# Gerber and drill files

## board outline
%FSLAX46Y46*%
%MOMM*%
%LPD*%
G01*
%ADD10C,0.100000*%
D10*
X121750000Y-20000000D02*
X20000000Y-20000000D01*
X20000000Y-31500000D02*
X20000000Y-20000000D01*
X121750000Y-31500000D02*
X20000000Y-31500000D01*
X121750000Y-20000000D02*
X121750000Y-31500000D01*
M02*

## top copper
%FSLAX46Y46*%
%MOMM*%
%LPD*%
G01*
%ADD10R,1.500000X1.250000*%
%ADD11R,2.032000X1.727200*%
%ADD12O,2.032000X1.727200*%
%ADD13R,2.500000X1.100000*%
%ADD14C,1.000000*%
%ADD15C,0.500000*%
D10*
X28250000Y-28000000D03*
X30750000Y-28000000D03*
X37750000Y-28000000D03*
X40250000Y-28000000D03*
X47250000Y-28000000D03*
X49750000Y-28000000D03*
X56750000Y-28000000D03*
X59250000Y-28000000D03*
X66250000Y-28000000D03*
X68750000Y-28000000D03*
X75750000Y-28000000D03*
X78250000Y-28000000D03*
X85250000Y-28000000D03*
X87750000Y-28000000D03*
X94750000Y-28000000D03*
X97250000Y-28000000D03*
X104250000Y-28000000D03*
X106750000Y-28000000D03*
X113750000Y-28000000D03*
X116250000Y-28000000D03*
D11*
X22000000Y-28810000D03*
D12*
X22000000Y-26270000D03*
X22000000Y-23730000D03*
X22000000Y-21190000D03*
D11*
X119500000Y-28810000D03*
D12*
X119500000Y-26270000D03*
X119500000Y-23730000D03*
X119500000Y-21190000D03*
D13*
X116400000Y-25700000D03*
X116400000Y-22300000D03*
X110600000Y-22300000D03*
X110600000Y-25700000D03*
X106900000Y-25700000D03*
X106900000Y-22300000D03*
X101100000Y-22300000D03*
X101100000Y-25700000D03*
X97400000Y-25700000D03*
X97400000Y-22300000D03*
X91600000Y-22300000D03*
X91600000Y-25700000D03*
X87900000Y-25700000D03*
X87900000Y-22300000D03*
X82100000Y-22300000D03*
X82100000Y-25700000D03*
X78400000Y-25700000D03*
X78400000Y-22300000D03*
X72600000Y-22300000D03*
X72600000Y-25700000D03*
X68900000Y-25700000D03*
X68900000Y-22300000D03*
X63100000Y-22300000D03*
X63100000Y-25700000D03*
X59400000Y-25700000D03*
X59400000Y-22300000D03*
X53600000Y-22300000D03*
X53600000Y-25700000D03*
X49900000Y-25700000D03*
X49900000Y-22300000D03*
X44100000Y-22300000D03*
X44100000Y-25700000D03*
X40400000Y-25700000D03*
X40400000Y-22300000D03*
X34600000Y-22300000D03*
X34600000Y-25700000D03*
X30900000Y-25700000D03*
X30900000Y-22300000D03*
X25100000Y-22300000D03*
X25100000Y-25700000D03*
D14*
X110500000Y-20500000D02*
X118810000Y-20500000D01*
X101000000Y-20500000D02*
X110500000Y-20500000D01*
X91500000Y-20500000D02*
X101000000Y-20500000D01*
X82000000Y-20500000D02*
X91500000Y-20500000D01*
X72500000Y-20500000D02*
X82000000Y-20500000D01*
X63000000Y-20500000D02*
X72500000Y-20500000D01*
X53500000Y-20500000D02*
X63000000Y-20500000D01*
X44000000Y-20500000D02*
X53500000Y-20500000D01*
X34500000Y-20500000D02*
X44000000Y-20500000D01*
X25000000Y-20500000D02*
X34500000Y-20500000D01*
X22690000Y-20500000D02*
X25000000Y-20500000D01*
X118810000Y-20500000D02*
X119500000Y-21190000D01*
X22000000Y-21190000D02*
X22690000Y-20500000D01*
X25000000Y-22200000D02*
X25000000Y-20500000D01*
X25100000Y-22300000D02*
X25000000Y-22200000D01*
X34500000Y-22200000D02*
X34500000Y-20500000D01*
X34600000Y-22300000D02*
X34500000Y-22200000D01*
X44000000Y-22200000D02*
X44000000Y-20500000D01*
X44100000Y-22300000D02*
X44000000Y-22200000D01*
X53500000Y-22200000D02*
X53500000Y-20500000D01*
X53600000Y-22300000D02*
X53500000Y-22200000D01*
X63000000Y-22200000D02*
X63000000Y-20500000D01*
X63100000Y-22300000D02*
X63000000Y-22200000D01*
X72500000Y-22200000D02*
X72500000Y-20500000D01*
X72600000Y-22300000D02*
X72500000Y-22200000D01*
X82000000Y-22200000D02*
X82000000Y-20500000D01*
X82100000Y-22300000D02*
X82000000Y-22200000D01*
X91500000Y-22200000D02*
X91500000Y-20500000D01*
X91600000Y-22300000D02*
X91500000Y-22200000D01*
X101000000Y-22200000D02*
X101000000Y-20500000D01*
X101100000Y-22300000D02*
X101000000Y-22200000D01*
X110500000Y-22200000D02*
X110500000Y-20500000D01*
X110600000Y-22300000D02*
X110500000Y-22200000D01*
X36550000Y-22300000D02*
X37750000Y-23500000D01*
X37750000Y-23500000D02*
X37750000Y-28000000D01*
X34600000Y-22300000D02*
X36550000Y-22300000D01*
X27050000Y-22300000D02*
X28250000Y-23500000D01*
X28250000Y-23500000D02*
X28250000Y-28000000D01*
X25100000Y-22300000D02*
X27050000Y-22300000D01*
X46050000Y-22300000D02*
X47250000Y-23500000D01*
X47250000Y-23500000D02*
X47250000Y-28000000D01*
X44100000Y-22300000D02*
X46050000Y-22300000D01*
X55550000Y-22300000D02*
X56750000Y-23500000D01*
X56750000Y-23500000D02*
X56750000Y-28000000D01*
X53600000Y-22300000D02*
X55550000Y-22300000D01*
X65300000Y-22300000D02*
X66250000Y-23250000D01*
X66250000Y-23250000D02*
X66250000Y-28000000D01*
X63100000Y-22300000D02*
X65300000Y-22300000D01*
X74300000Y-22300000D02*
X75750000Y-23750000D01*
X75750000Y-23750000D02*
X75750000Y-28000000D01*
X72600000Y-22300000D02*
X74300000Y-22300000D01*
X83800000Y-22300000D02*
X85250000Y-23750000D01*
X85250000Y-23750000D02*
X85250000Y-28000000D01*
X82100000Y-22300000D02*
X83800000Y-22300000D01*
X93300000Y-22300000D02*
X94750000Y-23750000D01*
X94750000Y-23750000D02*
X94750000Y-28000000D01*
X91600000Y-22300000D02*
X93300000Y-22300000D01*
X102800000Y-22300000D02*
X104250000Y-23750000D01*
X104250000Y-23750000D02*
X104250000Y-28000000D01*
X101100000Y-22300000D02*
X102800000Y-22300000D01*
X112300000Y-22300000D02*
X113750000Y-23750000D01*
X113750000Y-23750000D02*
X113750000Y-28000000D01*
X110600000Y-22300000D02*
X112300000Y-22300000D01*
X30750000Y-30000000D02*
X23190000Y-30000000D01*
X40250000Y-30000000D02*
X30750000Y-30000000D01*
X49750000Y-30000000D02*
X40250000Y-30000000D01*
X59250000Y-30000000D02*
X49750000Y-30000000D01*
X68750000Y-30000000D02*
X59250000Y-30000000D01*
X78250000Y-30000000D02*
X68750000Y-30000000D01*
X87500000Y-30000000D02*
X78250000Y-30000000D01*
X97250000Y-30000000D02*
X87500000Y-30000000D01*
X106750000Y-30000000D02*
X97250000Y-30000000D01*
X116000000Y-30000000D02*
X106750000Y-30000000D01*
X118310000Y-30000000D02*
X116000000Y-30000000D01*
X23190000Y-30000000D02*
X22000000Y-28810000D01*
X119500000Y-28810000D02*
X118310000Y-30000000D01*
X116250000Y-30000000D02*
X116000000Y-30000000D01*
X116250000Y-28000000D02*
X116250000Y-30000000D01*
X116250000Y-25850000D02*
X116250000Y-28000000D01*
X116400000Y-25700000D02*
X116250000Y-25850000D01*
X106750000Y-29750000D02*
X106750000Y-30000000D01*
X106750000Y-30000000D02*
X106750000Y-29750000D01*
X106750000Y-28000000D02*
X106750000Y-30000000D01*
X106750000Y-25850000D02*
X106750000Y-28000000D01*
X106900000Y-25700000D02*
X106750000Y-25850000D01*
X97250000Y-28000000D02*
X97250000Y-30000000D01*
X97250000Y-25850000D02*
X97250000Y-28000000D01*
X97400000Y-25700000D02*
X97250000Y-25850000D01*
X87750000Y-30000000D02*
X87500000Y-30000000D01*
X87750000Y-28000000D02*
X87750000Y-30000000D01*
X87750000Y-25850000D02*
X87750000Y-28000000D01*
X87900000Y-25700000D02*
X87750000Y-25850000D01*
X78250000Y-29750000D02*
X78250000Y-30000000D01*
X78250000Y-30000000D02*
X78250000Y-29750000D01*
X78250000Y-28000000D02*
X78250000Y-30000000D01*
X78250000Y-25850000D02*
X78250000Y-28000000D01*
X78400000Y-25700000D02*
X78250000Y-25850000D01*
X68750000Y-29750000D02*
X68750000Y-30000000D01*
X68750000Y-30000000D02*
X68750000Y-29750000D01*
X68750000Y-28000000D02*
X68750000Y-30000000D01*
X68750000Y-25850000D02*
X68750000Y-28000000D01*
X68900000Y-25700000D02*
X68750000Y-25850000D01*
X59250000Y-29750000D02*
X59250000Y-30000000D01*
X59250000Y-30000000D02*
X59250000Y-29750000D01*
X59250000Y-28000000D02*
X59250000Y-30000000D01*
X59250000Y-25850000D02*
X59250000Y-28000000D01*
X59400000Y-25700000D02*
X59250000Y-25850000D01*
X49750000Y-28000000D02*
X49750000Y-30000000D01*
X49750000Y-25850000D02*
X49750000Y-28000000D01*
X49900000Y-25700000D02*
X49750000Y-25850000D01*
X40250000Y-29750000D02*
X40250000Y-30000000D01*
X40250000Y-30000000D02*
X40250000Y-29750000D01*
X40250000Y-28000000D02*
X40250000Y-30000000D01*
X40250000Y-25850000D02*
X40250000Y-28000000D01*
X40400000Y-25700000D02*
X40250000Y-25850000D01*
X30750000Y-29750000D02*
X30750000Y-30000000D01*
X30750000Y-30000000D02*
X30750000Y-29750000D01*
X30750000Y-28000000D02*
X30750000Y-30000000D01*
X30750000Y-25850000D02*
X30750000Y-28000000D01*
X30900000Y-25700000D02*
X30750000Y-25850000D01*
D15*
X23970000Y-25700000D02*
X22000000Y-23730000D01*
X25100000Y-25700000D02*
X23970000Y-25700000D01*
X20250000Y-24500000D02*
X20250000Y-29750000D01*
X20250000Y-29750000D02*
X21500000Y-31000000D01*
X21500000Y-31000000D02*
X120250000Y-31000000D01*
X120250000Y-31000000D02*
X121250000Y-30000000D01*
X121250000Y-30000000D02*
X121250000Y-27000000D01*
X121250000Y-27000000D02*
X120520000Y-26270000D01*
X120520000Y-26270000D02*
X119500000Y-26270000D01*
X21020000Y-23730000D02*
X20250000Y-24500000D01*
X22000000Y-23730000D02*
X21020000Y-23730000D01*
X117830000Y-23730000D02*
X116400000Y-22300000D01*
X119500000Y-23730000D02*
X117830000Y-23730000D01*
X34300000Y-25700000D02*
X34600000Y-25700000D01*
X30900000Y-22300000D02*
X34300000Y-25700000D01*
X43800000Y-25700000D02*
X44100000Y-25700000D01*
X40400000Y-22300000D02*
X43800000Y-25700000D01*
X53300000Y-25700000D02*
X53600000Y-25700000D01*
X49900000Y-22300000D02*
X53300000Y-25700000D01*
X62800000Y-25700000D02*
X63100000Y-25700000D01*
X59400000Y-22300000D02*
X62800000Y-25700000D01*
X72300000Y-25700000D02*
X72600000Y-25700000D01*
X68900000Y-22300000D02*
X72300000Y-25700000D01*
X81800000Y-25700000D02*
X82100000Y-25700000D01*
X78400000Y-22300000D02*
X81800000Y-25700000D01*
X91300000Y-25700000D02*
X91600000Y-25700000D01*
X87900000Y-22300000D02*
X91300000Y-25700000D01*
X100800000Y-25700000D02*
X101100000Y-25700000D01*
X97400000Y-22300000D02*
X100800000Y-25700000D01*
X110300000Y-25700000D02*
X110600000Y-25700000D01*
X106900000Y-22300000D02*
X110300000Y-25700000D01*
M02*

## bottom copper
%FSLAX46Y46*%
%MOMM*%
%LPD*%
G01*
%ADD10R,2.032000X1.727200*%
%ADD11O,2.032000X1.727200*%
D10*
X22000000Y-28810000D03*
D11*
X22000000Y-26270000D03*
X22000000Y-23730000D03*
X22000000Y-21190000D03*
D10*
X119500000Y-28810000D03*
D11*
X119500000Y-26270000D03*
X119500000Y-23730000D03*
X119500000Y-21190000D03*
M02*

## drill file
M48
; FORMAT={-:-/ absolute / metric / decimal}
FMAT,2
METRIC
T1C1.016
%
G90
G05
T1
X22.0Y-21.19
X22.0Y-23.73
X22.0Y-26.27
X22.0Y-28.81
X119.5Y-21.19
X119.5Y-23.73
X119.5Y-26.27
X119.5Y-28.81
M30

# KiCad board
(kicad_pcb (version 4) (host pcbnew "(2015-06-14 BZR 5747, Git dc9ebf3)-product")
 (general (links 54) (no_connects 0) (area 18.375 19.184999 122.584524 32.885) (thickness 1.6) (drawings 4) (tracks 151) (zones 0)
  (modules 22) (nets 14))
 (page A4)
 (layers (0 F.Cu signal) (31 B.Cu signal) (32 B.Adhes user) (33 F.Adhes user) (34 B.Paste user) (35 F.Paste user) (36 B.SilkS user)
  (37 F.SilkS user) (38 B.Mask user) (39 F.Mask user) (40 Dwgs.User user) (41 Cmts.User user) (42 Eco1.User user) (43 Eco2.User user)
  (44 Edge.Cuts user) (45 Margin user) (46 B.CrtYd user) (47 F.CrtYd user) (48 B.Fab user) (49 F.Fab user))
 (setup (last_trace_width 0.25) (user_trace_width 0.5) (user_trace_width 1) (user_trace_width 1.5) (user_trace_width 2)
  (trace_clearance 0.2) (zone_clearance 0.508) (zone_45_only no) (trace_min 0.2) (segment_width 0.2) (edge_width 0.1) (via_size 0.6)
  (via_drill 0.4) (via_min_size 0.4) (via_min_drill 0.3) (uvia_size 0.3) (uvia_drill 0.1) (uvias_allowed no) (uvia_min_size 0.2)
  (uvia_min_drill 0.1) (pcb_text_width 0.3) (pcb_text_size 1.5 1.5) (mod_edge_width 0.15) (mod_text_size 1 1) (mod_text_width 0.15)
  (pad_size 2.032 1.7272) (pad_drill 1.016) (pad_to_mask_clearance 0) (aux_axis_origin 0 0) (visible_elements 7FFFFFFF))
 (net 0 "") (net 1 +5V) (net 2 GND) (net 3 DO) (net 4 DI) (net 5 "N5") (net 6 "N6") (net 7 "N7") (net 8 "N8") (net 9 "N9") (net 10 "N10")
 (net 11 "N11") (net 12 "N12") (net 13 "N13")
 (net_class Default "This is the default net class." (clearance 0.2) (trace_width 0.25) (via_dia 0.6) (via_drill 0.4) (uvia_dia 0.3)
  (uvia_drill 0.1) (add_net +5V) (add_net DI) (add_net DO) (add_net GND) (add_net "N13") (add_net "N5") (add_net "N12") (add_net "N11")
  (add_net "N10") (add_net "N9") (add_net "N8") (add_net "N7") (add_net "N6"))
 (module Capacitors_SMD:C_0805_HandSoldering (layer F.Cu) (at 29.5 28)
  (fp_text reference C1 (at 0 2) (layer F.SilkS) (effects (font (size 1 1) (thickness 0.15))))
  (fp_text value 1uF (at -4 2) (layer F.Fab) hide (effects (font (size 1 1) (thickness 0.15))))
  (pad 1 smd rect (at -1.25 0) (size 1.5 1.25) (layers F.Cu F.Paste F.Mask) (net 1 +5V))
  (pad 2 smd rect (at 1.25 0) (size 1.5 1.25) (layers F.Cu F.Paste F.Mask) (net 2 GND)))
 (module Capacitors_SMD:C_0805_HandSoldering (layer F.Cu) (at 39 28)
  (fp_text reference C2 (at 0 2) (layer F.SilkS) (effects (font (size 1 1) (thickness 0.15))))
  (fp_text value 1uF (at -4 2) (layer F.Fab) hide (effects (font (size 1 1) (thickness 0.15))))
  (pad 1 smd rect (at -1.25 0) (size 1.5 1.25) (layers F.Cu F.Paste F.Mask) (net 1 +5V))
  (pad 2 smd rect (at 1.25 0) (size 1.5 1.25) (layers F.Cu F.Paste F.Mask) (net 2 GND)))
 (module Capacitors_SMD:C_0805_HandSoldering (layer F.Cu) (at 48.5 28)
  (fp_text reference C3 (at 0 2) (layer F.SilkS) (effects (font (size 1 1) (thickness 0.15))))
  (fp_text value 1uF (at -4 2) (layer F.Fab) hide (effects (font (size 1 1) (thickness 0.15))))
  (pad 1 smd rect (at -1.25 0) (size 1.5 1.25) (layers F.Cu F.Paste F.Mask) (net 1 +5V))
  (pad 2 smd rect (at 1.25 0) (size 1.5 1.25) (layers F.Cu F.Paste F.Mask) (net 2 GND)))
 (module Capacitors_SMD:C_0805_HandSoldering (layer F.Cu) (at 58 28)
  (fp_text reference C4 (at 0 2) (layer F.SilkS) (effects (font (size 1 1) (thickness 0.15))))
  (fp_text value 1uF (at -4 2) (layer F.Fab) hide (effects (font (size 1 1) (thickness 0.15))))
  (pad 1 smd rect (at -1.25 0) (size 1.5 1.25) (layers F.Cu F.Paste F.Mask) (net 1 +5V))
  (pad 2 smd rect (at 1.25 0) (size 1.5 1.25) (layers F.Cu F.Paste F.Mask) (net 2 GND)))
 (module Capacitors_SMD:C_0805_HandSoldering (layer F.Cu) (at 67.5 28)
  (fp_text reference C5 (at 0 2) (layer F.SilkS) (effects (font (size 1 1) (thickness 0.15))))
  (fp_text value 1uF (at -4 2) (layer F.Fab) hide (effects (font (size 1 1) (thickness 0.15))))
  (pad 1 smd rect (at -1.25 0) (size 1.5 1.25) (layers F.Cu F.Paste F.Mask) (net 1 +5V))
  (pad 2 smd rect (at 1.25 0) (size 1.5 1.25) (layers F.Cu F.Paste F.Mask) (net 2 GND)))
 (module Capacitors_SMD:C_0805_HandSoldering (layer F.Cu) (at 77 28)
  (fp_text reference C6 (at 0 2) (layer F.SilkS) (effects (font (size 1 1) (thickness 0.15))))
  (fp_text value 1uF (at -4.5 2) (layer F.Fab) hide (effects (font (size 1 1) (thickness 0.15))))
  (pad 1 smd rect (at -1.25 0) (size 1.5 1.25) (layers F.Cu F.Paste F.Mask) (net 1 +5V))
  (pad 2 smd rect (at 1.25 0) (size 1.5 1.25) (layers F.Cu F.Paste F.Mask) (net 2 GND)))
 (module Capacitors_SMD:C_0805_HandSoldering (layer F.Cu) (at 86.5 28)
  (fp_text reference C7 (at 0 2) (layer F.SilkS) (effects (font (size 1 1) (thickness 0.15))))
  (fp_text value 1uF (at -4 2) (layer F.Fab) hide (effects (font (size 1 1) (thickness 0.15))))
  (pad 1 smd rect (at -1.25 0) (size 1.5 1.25) (layers F.Cu F.Paste F.Mask) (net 1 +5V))
  (pad 2 smd rect (at 1.25 0) (size 1.5 1.25) (layers F.Cu F.Paste F.Mask) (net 2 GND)))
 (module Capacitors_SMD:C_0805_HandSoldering (layer F.Cu) (at 96 28)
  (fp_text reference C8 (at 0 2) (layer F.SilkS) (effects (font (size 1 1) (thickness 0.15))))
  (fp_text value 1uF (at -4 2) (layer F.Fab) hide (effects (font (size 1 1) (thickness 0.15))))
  (pad 1 smd rect (at -1.25 0) (size 1.5 1.25) (layers F.Cu F.Paste F.Mask) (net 1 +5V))
  (pad 2 smd rect (at 1.25 0) (size 1.5 1.25) (layers F.Cu F.Paste F.Mask) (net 2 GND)))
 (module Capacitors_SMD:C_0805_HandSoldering (layer F.Cu) (at 105.5 28)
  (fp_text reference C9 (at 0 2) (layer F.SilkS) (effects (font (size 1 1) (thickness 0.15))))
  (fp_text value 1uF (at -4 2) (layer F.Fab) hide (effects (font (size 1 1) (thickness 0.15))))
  (pad 1 smd rect (at -1.25 0) (size 1.5 1.25) (layers F.Cu F.Paste F.Mask) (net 1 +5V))
  (pad 2 smd rect (at 1.25 0) (size 1.5 1.25) (layers F.Cu F.Paste F.Mask) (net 2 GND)))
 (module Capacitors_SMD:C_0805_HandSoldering (layer F.Cu) (at 115 28)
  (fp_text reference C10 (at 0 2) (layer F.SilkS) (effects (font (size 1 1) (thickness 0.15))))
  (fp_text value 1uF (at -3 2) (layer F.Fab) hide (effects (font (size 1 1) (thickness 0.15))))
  (pad 1 smd rect (at -1.25 0) (size 1.5 1.25) (layers F.Cu F.Paste F.Mask) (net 1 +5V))
  (pad 2 smd rect (at 1.25 0) (size 1.5 1.25) (layers F.Cu F.Paste F.Mask) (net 2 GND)))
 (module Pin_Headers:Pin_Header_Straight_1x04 (layer F.Cu) (at 22 28.81 180)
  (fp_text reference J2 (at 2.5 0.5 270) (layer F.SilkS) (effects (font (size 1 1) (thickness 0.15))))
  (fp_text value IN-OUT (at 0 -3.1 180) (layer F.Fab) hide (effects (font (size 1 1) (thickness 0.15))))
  (pad 1 thru_hole rect (at 0 0 180) (size 2.032 1.7272) (drill 1.016) (layers *.Cu *.Mask F.SilkS) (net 2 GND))
  (pad 2 thru_hole oval (at 0 2.54 180) (size 2.032 1.7272) (drill 1.016) (layers *.Cu *.Mask F.SilkS))
  (pad 3 thru_hole oval (at 0 5.08 180) (size 2.032 1.7272) (drill 1.016) (layers *.Cu *.Mask F.SilkS) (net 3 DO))
  (pad 4 thru_hole oval (at 0 7.62 180) (size 2.032 1.7272) (drill 1.016) (layers *.Cu *.Mask F.SilkS) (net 1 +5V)))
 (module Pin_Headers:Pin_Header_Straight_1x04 (layer F.Cu) (at 119.5 28.81 180)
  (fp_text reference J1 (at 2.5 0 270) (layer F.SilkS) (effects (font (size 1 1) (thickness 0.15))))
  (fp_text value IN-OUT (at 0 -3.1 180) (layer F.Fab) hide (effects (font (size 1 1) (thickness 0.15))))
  (pad 1 thru_hole rect (at 0 0 180) (size 2.032 1.7272) (drill 1.016) (layers *.Cu *.Mask F.SilkS) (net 2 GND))
  (pad 2 thru_hole oval (at 0 2.54 180) (size 2.032 1.7272) (drill 1.016) (layers *.Cu *.Mask F.SilkS) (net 3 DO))
  (pad 3 thru_hole oval (at 0 5.08 180) (size 2.032 1.7272) (drill 1.016) (layers *.Cu *.Mask F.SilkS) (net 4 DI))
  (pad 4 thru_hole oval (at 0 7.62 180) (size 2.032 1.7272) (drill 1.016) (layers *.Cu *.Mask F.SilkS) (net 1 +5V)))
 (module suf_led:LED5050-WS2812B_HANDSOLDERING (layer F.Cu) (at 113.5 24 90)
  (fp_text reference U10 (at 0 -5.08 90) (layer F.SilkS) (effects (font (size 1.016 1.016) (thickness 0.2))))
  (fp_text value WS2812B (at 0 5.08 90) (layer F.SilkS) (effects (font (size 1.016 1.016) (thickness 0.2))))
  (pad 3 smd rect (at -1.7 2.9 90) (size 1.1 2.5) (layers F.Cu F.Paste F.Mask) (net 2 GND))
  (pad 4 smd rect (at 1.7 2.9 90) (size 1.1 2.5) (layers F.Cu F.Paste F.Mask) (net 4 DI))
  (pad 1 smd rect (at 1.7 -2.9 90) (size 1.1 2.5) (layers F.Cu F.Paste F.Mask) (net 1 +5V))
  (pad 2 smd rect (at -1.7 -2.9 90) (size 1.1 2.5) (layers F.Cu F.Paste F.Mask) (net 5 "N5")))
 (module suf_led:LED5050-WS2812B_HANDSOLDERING (layer F.Cu) (at 104 24 90)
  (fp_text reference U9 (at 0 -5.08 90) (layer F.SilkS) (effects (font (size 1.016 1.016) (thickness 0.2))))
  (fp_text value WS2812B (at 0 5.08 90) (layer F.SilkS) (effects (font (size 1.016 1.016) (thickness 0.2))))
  (pad 3 smd rect (at -1.7 2.9 90) (size 1.1 2.5) (layers F.Cu F.Paste F.Mask) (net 2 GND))
  (pad 4 smd rect (at 1.7 2.9 90) (size 1.1 2.5) (layers F.Cu F.Paste F.Mask) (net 5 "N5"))
  (pad 1 smd rect (at 1.7 -2.9 90) (size 1.1 2.5) (layers F.Cu F.Paste F.Mask) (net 1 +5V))
  (pad 2 smd rect (at -1.7 -2.9 90) (size 1.1 2.5) (layers F.Cu F.Paste F.Mask) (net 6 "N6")))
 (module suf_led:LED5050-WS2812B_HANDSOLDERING (layer F.Cu) (at 94.5 24 90)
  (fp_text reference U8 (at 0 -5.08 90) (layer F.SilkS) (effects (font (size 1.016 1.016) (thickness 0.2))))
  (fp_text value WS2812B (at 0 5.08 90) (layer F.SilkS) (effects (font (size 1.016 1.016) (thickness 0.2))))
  (pad 3 smd rect (at -1.7 2.9 90) (size 1.1 2.5) (layers F.Cu F.Paste F.Mask) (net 2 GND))
  (pad 4 smd rect (at 1.7 2.9 90) (size 1.1 2.5) (layers F.Cu F.Paste F.Mask) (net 6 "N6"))
  (pad 1 smd rect (at 1.7 -2.9 90) (size 1.1 2.5) (layers F.Cu F.Paste F.Mask) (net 1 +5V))
  (pad 2 smd rect (at -1.7 -2.9 90) (size 1.1 2.5) (layers F.Cu F.Paste F.Mask) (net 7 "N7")))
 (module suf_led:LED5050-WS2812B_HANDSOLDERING (layer F.Cu) (at 85 24 90)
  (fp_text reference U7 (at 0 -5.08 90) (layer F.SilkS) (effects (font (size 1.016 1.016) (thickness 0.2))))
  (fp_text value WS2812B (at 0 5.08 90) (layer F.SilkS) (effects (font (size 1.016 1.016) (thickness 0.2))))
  (pad 3 smd rect (at -1.7 2.9 90) (size 1.1 2.5) (layers F.Cu F.Paste F.Mask) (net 2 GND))
  (pad 4 smd rect (at 1.7 2.9 90) (size 1.1 2.5) (layers F.Cu F.Paste F.Mask) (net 7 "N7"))
  (pad 1 smd rect (at 1.7 -2.9 90) (size 1.1 2.5) (layers F.Cu F.Paste F.Mask) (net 1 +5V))
  (pad 2 smd rect (at -1.7 -2.9 90) (size 1.1 2.5) (layers F.Cu F.Paste F.Mask) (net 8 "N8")))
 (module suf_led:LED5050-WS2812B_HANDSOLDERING (layer F.Cu) (at 75.5 24 90)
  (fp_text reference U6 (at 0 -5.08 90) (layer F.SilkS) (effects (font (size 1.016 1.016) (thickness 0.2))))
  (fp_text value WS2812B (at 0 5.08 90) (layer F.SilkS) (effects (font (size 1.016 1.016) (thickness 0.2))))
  (pad 3 smd rect (at -1.7 2.9 90) (size 1.1 2.5) (layers F.Cu F.Paste F.Mask) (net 2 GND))
  (pad 4 smd rect (at 1.7 2.9 90) (size 1.1 2.5) (layers F.Cu F.Paste F.Mask) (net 8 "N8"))
  (pad 1 smd rect (at 1.7 -2.9 90) (size 1.1 2.5) (layers F.Cu F.Paste F.Mask) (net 1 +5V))
  (pad 2 smd rect (at -1.7 -2.9 90) (size 1.1 2.5) (layers F.Cu F.Paste F.Mask) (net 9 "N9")))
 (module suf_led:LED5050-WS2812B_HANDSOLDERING (layer F.Cu) (at 66 24 90)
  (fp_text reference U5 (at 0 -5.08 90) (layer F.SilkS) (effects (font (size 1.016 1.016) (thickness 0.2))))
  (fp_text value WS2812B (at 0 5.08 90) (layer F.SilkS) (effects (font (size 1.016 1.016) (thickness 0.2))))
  (pad 3 smd rect (at -1.7 2.9 90) (size 1.1 2.5) (layers F.Cu F.Paste F.Mask) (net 2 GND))
  (pad 4 smd rect (at 1.7 2.9 90) (size 1.1 2.5) (layers F.Cu F.Paste F.Mask) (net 9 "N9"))
  (pad 1 smd rect (at 1.7 -2.9 90) (size 1.1 2.5) (layers F.Cu F.Paste F.Mask) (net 1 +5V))
  (pad 2 smd rect (at -1.7 -2.9 90) (size 1.1 2.5) (layers F.Cu F.Paste F.Mask) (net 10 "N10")))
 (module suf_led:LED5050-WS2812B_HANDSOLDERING (layer F.Cu) (at 56.5 24 90)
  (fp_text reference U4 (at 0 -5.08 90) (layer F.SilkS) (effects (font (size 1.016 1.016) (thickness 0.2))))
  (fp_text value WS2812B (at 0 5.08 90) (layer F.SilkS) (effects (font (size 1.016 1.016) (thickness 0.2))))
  (pad 3 smd rect (at -1.7 2.9 90) (size 1.1 2.5) (layers F.Cu F.Paste F.Mask) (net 2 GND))
  (pad 4 smd rect (at 1.7 2.9 90) (size 1.1 2.5) (layers F.Cu F.Paste F.Mask) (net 10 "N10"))
  (pad 1 smd rect (at 1.7 -2.9 90) (size 1.1 2.5) (layers F.Cu F.Paste F.Mask) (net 1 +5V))
  (pad 2 smd rect (at -1.7 -2.9 90) (size 1.1 2.5) (layers F.Cu F.Paste F.Mask) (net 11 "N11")))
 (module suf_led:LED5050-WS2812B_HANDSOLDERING (layer F.Cu) (at 47 24 90)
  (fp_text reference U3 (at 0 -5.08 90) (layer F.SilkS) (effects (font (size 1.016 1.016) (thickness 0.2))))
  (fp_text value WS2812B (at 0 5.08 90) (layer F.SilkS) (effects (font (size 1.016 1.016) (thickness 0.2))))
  (pad 3 smd rect (at -1.7 2.9 90) (size 1.1 2.5) (layers F.Cu F.Paste F.Mask) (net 2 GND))
  (pad 4 smd rect (at 1.7 2.9 90) (size 1.1 2.5) (layers F.Cu F.Paste F.Mask) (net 11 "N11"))
  (pad 1 smd rect (at 1.7 -2.9 90) (size 1.1 2.5) (layers F.Cu F.Paste F.Mask) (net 1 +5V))
  (pad 2 smd rect (at -1.7 -2.9 90) (size 1.1 2.5) (layers F.Cu F.Paste F.Mask) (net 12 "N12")))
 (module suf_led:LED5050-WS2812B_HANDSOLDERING (layer F.Cu) (at 37.5 24 90)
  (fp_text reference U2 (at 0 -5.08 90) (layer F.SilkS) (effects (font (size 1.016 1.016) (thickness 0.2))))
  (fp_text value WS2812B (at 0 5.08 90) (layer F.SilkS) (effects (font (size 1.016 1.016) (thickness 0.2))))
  (pad 3 smd rect (at -1.7 2.9 90) (size 1.1 2.5) (layers F.Cu F.Paste F.Mask) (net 2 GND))
  (pad 4 smd rect (at 1.7 2.9 90) (size 1.1 2.5) (layers F.Cu F.Paste F.Mask) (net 12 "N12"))
  (pad 1 smd rect (at 1.7 -2.9 90) (size 1.1 2.5) (layers F.Cu F.Paste F.Mask) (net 1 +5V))
  (pad 2 smd rect (at -1.7 -2.9 90) (size 1.1 2.5) (layers F.Cu F.Paste F.Mask) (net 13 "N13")))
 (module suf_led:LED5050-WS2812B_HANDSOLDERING (layer F.Cu) (at 28 24 90)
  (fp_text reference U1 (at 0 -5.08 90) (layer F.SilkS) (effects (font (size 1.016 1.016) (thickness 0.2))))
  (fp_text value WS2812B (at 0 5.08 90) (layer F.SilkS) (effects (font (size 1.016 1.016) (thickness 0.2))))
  (pad 3 smd rect (at -1.7 2.9 90) (size 1.1 2.5) (layers F.Cu F.Paste F.Mask) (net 2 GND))
  (pad 4 smd rect (at 1.7 2.9 90) (size 1.1 2.5) (layers F.Cu F.Paste F.Mask) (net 13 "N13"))
  (pad 1 smd rect (at 1.7 -2.9 90) (size 1.1 2.5) (layers F.Cu F.Paste F.Mask) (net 1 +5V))
  (pad 2 smd rect (at -1.7 -2.9 90) (size 1.1 2.5) (layers F.Cu F.Paste F.Mask) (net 3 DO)))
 (gr_line (start 121.75 20) (end 20 20) (angle 90) (layer Edge.Cuts) (width 0.1))
 (gr_line (start 20 31.5) (end 20 20) (angle 90) (layer Edge.Cuts) (width 0.1))
 (gr_line (start 121.75 31.5) (end 20 31.5) (angle 90) (layer Edge.Cuts) (width 0.1))
 (gr_line (start 121.75 20) (end 121.75 31.5) (angle 90) (layer Edge.Cuts) (width 0.1))
 (segment (start 110.5 20.5) (end 118.81 20.5) (width 1) (layer F.Cu) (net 1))
 (segment (start 101 20.5) (end 110.5 20.5) (width 1) (layer F.Cu) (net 1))
 (segment (start 91.5 20.5) (end 101 20.5) (width 1) (layer F.Cu) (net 1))
 (segment (start 82 20.5) (end 91.5 20.5) (width 1) (layer F.Cu) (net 1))
 (segment (start 72.5 20.5) (end 82 20.5) (width 1) (layer F.Cu) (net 1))
 (segment (start 63 20.5) (end 72.5 20.5) (width 1) (layer F.Cu) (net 1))
 (segment (start 53.5 20.5) (end 63 20.5) (width 1) (layer F.Cu) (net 1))
 (segment (start 44 20.5) (end 53.5 20.5) (width 1) (layer F.Cu) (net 1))
 (segment (start 34.5 20.5) (end 44 20.5) (width 1) (layer F.Cu) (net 1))
 (segment (start 25 20.5) (end 34.5 20.5) (width 1) (layer F.Cu) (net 1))
 (segment (start 22.69 20.5) (end 25 20.5) (width 1) (layer F.Cu) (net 1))
 (segment (start 118.81 20.5) (end 119.5 21.19) (width 1) (layer F.Cu) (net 1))
 (segment (start 22 21.19) (end 22.69 20.5) (width 1) (layer F.Cu) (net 1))
 (segment (start 25 22.2) (end 25 20.5) (width 1) (layer F.Cu) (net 1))
 (segment (start 25.1 22.3) (end 25 22.2) (width 1) (layer F.Cu) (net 1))
 (segment (start 34.5 22.2) (end 34.5 20.5) (width 1) (layer F.Cu) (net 1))
 (segment (start 34.6 22.3) (end 34.5 22.2) (width 1) (layer F.Cu) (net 1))
 (segment (start 44 22.2) (end 44 20.5) (width 1) (layer F.Cu) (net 1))
 (segment (start 44.1 22.3) (end 44 22.2) (width 1) (layer F.Cu) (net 1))
 (segment (start 53.5 22.2) (end 53.5 20.5) (width 1) (layer F.Cu) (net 1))
 (segment (start 53.6 22.3) (end 53.5 22.2) (width 1) (layer F.Cu) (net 1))
 (segment (start 63 22.2) (end 63 20.5) (width 1) (layer F.Cu) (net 1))
 (segment (start 63.1 22.3) (end 63 22.2) (width 1) (layer F.Cu) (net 1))
 (segment (start 72.5 22.2) (end 72.5 20.5) (width 1) (layer F.Cu) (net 1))
 (segment (start 72.6 22.3) (end 72.5 22.2) (width 1) (layer F.Cu) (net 1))
 (segment (start 82 22.2) (end 82 20.5) (width 1) (layer F.Cu) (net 1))
 (segment (start 82.1 22.3) (end 82 22.2) (width 1) (layer F.Cu) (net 1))
 (segment (start 91.5 22.2) (end 91.5 20.5) (width 1) (layer F.Cu) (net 1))
 (segment (start 91.6 22.3) (end 91.5 22.2) (width 1) (layer F.Cu) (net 1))
 (segment (start 101 22.2) (end 101 20.5) (width 1) (layer F.Cu) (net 1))
 (segment (start 101.1 22.3) (end 101 22.2) (width 1) (layer F.Cu) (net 1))
 (segment (start 110.5 22.2) (end 110.5 20.5) (width 1) (layer F.Cu) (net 1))
 (segment (start 110.6 22.3) (end 110.5 22.2) (width 1) (layer F.Cu) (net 1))
 (segment (start 36.55 22.3) (end 37.75 23.5) (width 1) (layer F.Cu) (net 1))
 (segment (start 37.75 23.5) (end 37.75 28) (width 1) (layer F.Cu) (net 1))
 (segment (start 34.6 22.3) (end 36.55 22.3) (width 1) (layer F.Cu) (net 1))
 (segment (start 27.05 22.3) (end 28.25 23.5) (width 1) (layer F.Cu) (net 1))
 (segment (start 28.25 23.5) (end 28.25 28) (width 1) (layer F.Cu) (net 1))
 (segment (start 25.1 22.3) (end 27.05 22.3) (width 1) (layer F.Cu) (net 1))
 (segment (start 46.05 22.3) (end 47.25 23.5) (width 1) (layer F.Cu) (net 1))
 (segment (start 47.25 23.5) (end 47.25 28) (width 1) (layer F.Cu) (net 1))
 (segment (start 44.1 22.3) (end 46.05 22.3) (width 1) (layer F.Cu) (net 1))
 (segment (start 55.55 22.3) (end 56.75 23.5) (width 1) (layer F.Cu) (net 1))
 (segment (start 56.75 23.5) (end 56.75 28) (width 1) (layer F.Cu) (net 1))
 (segment (start 53.6 22.3) (end 55.55 22.3) (width 1) (layer F.Cu) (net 1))
 (segment (start 65.3 22.3) (end 66.25 23.25) (width 1) (layer F.Cu) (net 1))
 (segment (start 66.25 23.25) (end 66.25 28) (width 1) (layer F.Cu) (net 1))
 (segment (start 63.1 22.3) (end 65.3 22.3) (width 1) (layer F.Cu) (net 1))
 (segment (start 74.3 22.3) (end 75.75 23.75) (width 1) (layer F.Cu) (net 1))
 (segment (start 75.75 23.75) (end 75.75 28) (width 1) (layer F.Cu) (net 1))
 (segment (start 72.6 22.3) (end 74.3 22.3) (width 1) (layer F.Cu) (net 1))
 (segment (start 83.8 22.3) (end 85.25 23.75) (width 1) (layer F.Cu) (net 1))
 (segment (start 85.25 23.75) (end 85.25 28) (width 1) (layer F.Cu) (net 1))
 (segment (start 82.1 22.3) (end 83.8 22.3) (width 1) (layer F.Cu) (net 1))
 (segment (start 93.3 22.3) (end 94.75 23.75) (width 1) (layer F.Cu) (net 1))
 (segment (start 94.75 23.75) (end 94.75 28) (width 1) (layer F.Cu) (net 1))
 (segment (start 91.6 22.3) (end 93.3 22.3) (width 1) (layer F.Cu) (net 1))
 (segment (start 102.8 22.3) (end 104.25 23.75) (width 1) (layer F.Cu) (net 1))
 (segment (start 104.25 23.75) (end 104.25 28) (width 1) (layer F.Cu) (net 1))
 (segment (start 101.1 22.3) (end 102.8 22.3) (width 1) (layer F.Cu) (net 1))
 (segment (start 112.3 22.3) (end 113.75 23.75) (width 1) (layer F.Cu) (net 1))
 (segment (start 113.75 23.75) (end 113.75 28) (width 1) (layer F.Cu) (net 1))
 (segment (start 110.6 22.3) (end 112.3 22.3) (width 1) (layer F.Cu) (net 1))
 (segment (start 30.75 30) (end 23.19 30) (width 1) (layer F.Cu) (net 2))
 (segment (start 40.25 30) (end 30.75 30) (width 1) (layer F.Cu) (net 2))
 (segment (start 49.75 30) (end 40.25 30) (width 1) (layer F.Cu) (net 2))
 (segment (start 59.25 30) (end 49.75 30) (width 1) (layer F.Cu) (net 2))
 (segment (start 68.75 30) (end 59.25 30) (width 1) (layer F.Cu) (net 2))
 (segment (start 78.25 30) (end 68.75 30) (width 1) (layer F.Cu) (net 2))
 (segment (start 87.5 30) (end 78.25 30) (width 1) (layer F.Cu) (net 2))
 (segment (start 97.25 30) (end 87.5 30) (width 1) (layer F.Cu) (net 2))
 (segment (start 106.75 30) (end 97.25 30) (width 1) (layer F.Cu) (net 2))
 (segment (start 116 30) (end 106.75 30) (width 1) (layer F.Cu) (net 2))
 (segment (start 118.31 30) (end 116 30) (width 1) (layer F.Cu) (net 2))
 (segment (start 23.19 30) (end 22 28.81) (width 1) (layer F.Cu) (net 2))
 (segment (start 119.5 28.81) (end 118.31 30) (width 1) (layer F.Cu) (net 2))
 (segment (start 116.25 30) (end 116 30) (width 1) (layer F.Cu) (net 2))
 (segment (start 116.25 28) (end 116.25 30) (width 1) (layer F.Cu) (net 2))
 (segment (start 116.25 25.85) (end 116.25 28) (width 1) (layer F.Cu) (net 2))
 (segment (start 116.4 25.7) (end 116.25 25.85) (width 1) (layer F.Cu) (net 2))
 (segment (start 106.75 29.75) (end 106.75 30) (width 1) (layer F.Cu) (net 2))
 (segment (start 106.75 30) (end 106.75 29.75) (width 1) (layer F.Cu) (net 2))
 (segment (start 106.75 28) (end 106.75 30) (width 1) (layer F.Cu) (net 2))
 (segment (start 106.75 25.85) (end 106.75 28) (width 1) (layer F.Cu) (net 2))
 (segment (start 106.9 25.7) (end 106.75 25.85) (width 1) (layer F.Cu) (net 2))
 (segment (start 97.25 28) (end 97.25 30) (width 1) (layer F.Cu) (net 2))
 (segment (start 97.25 25.85) (end 97.25 28) (width 1) (layer F.Cu) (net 2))
 (segment (start 97.4 25.7) (end 97.25 25.85) (width 1) (layer F.Cu) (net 2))
 (segment (start 87.75 30) (end 87.5 30) (width 1) (layer F.Cu) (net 2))
 (segment (start 87.75 28) (end 87.75 30) (width 1) (layer F.Cu) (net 2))
 (segment (start 87.75 25.85) (end 87.75 28) (width 1) (layer F.Cu) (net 2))
 (segment (start 87.9 25.7) (end 87.75 25.85) (width 1) (layer F.Cu) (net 2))
 (segment (start 78.25 29.75) (end 78.25 30) (width 1) (layer F.Cu) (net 2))
 (segment (start 78.25 30) (end 78.25 29.75) (width 1) (layer F.Cu) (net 2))
 (segment (start 78.25 28) (end 78.25 30) (width 1) (layer F.Cu) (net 2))
 (segment (start 78.25 25.85) (end 78.25 28) (width 1) (layer F.Cu) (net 2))
 (segment (start 78.4 25.7) (end 78.25 25.85) (width 1) (layer F.Cu) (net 2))
 (segment (start 68.75 29.75) (end 68.75 30) (width 1) (layer F.Cu) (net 2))
 (segment (start 68.75 30) (end 68.75 29.75) (width 1) (layer F.Cu) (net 2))
 (segment (start 68.75 28) (end 68.75 30) (width 1) (layer F.Cu) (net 2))
 (segment (start 68.75 25.85) (end 68.75 28) (width 1) (layer F.Cu) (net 2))
 (segment (start 68.9 25.7) (end 68.75 25.85) (width 1) (layer F.Cu) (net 2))
 (segment (start 59.25 29.75) (end 59.25 30) (width 1) (layer F.Cu) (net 2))
 (segment (start 59.25 30) (end 59.25 29.75) (width 1) (layer F.Cu) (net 2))
 (segment (start 59.25 28) (end 59.25 30) (width 1) (layer F.Cu) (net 2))
 (segment (start 59.25 25.85) (end 59.25 28) (width 1) (layer F.Cu) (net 2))
 (segment (start 59.4 25.7) (end 59.25 25.85) (width 1) (layer F.Cu) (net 2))
 (segment (start 49.75 28) (end 49.75 30) (width 1) (layer F.Cu) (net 2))
 (segment (start 49.75 25.85) (end 49.75 28) (width 1) (layer F.Cu) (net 2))
 (segment (start 49.9 25.7) (end 49.75 25.85) (width 1) (layer F.Cu) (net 2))
 (segment (start 40.25 29.75) (end 40.25 30) (width 1) (layer F.Cu) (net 2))
 (segment (start 40.25 30) (end 40.25 29.75) (width 1) (layer F.Cu) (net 2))
 (segment (start 40.25 28) (end 40.25 30) (width 1) (layer F.Cu) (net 2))
 (segment (start 40.25 25.85) (end 40.25 28) (width 1) (layer F.Cu) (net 2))
 (segment (start 40.4 25.7) (end 40.25 25.85) (width 1) (layer F.Cu) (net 2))
 (segment (start 30.75 29.75) (end 30.75 30) (width 1) (layer F.Cu) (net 2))
 (segment (start 30.75 30) (end 30.75 29.75) (width 1) (layer F.Cu) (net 2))
 (segment (start 30.75 28) (end 30.75 30) (width 1) (layer F.Cu) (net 2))
 (segment (start 30.75 25.85) (end 30.75 28) (width 1) (layer F.Cu) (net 2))
 (segment (start 30.9 25.7) (end 30.75 25.85) (width 1) (layer F.Cu) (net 2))
 (segment (start 23.97 25.7) (end 22 23.73) (width 0.5) (layer F.Cu) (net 3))
 (segment (start 25.1 25.7) (end 23.97 25.7) (width 0.5) (layer F.Cu) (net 3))
 (segment (start 20.25 24.5) (end 20.25 29.75) (width 0.5) (layer F.Cu) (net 3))
 (segment (start 20.25 29.75) (end 21.5 31) (width 0.5) (layer F.Cu) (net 3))
 (segment (start 21.5 31) (end 120.25 31) (width 0.5) (layer F.Cu) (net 3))
 (segment (start 120.25 31) (end 121.25 30) (width 0.5) (layer F.Cu) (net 3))
 (segment (start 121.25 30) (end 121.25 27) (width 0.5) (layer F.Cu) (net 3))
 (segment (start 121.25 27) (end 120.52 26.27) (width 0.5) (layer F.Cu) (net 3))
 (segment (start 120.52 26.27) (end 119.5 26.27) (width 0.5) (layer F.Cu) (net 3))
 (segment (start 21.02 23.73) (end 20.25 24.5) (width 0.5) (layer F.Cu) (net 3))
 (segment (start 22 23.73) (end 21.02 23.73) (width 0.5) (layer F.Cu) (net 3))
 (segment (start 117.83 23.73) (end 116.4 22.3) (width 0.5) (layer F.Cu) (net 4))
 (segment (start 119.5 23.73) (end 117.83 23.73) (width 0.5) (layer F.Cu) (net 4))
 (segment (start 34.3 25.7) (end 34.6 25.7) (width 0.5) (layer F.Cu) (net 13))
 (segment (start 30.9 22.3) (end 34.3 25.7) (width 0.5) (layer F.Cu) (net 13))
 (segment (start 43.8 25.7) (end 44.1 25.7) (width 0.5) (layer F.Cu) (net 12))
 (segment (start 40.4 22.3) (end 43.8 25.7) (width 0.5) (layer F.Cu) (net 12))
 (segment (start 53.3 25.7) (end 53.6 25.7) (width 0.5) (layer F.Cu) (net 11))
 (segment (start 49.9 22.3) (end 53.3 25.7) (width 0.5) (layer F.Cu) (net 11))
 (segment (start 62.8 25.7) (end 63.1 25.7) (width 0.5) (layer F.Cu) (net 10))
 (segment (start 59.4 22.3) (end 62.8 25.7) (width 0.5) (layer F.Cu) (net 10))
 (segment (start 72.3 25.7) (end 72.6 25.7) (width 0.5) (layer F.Cu) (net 9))
 (segment (start 68.9 22.3) (end 72.3 25.7) (width 0.5) (layer F.Cu) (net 9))
 (segment (start 81.8 25.7) (end 82.1 25.7) (width 0.5) (layer F.Cu) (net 8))
 (segment (start 78.4 22.3) (end 81.8 25.7) (width 0.5) (layer F.Cu) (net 8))
 (segment (start 91.3 25.7) (end 91.6 25.7) (width 0.5) (layer F.Cu) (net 7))
 (segment (start 87.9 22.3) (end 91.3 25.7) (width 0.5) (layer F.Cu) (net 7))
 (segment (start 100.8 25.7) (end 101.1 25.7) (width 0.5) (layer F.Cu) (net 6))
 (segment (start 97.4 22.3) (end 100.8 25.7) (width 0.5) (layer F.Cu) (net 6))
 (segment (start 110.3 25.7) (end 110.6 25.7) (width 0.5) (layer F.Cu) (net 5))
 (segment (start 106.9 22.3) (end 110.3 25.7) (width 0.5) (layer F.Cu) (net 5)))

